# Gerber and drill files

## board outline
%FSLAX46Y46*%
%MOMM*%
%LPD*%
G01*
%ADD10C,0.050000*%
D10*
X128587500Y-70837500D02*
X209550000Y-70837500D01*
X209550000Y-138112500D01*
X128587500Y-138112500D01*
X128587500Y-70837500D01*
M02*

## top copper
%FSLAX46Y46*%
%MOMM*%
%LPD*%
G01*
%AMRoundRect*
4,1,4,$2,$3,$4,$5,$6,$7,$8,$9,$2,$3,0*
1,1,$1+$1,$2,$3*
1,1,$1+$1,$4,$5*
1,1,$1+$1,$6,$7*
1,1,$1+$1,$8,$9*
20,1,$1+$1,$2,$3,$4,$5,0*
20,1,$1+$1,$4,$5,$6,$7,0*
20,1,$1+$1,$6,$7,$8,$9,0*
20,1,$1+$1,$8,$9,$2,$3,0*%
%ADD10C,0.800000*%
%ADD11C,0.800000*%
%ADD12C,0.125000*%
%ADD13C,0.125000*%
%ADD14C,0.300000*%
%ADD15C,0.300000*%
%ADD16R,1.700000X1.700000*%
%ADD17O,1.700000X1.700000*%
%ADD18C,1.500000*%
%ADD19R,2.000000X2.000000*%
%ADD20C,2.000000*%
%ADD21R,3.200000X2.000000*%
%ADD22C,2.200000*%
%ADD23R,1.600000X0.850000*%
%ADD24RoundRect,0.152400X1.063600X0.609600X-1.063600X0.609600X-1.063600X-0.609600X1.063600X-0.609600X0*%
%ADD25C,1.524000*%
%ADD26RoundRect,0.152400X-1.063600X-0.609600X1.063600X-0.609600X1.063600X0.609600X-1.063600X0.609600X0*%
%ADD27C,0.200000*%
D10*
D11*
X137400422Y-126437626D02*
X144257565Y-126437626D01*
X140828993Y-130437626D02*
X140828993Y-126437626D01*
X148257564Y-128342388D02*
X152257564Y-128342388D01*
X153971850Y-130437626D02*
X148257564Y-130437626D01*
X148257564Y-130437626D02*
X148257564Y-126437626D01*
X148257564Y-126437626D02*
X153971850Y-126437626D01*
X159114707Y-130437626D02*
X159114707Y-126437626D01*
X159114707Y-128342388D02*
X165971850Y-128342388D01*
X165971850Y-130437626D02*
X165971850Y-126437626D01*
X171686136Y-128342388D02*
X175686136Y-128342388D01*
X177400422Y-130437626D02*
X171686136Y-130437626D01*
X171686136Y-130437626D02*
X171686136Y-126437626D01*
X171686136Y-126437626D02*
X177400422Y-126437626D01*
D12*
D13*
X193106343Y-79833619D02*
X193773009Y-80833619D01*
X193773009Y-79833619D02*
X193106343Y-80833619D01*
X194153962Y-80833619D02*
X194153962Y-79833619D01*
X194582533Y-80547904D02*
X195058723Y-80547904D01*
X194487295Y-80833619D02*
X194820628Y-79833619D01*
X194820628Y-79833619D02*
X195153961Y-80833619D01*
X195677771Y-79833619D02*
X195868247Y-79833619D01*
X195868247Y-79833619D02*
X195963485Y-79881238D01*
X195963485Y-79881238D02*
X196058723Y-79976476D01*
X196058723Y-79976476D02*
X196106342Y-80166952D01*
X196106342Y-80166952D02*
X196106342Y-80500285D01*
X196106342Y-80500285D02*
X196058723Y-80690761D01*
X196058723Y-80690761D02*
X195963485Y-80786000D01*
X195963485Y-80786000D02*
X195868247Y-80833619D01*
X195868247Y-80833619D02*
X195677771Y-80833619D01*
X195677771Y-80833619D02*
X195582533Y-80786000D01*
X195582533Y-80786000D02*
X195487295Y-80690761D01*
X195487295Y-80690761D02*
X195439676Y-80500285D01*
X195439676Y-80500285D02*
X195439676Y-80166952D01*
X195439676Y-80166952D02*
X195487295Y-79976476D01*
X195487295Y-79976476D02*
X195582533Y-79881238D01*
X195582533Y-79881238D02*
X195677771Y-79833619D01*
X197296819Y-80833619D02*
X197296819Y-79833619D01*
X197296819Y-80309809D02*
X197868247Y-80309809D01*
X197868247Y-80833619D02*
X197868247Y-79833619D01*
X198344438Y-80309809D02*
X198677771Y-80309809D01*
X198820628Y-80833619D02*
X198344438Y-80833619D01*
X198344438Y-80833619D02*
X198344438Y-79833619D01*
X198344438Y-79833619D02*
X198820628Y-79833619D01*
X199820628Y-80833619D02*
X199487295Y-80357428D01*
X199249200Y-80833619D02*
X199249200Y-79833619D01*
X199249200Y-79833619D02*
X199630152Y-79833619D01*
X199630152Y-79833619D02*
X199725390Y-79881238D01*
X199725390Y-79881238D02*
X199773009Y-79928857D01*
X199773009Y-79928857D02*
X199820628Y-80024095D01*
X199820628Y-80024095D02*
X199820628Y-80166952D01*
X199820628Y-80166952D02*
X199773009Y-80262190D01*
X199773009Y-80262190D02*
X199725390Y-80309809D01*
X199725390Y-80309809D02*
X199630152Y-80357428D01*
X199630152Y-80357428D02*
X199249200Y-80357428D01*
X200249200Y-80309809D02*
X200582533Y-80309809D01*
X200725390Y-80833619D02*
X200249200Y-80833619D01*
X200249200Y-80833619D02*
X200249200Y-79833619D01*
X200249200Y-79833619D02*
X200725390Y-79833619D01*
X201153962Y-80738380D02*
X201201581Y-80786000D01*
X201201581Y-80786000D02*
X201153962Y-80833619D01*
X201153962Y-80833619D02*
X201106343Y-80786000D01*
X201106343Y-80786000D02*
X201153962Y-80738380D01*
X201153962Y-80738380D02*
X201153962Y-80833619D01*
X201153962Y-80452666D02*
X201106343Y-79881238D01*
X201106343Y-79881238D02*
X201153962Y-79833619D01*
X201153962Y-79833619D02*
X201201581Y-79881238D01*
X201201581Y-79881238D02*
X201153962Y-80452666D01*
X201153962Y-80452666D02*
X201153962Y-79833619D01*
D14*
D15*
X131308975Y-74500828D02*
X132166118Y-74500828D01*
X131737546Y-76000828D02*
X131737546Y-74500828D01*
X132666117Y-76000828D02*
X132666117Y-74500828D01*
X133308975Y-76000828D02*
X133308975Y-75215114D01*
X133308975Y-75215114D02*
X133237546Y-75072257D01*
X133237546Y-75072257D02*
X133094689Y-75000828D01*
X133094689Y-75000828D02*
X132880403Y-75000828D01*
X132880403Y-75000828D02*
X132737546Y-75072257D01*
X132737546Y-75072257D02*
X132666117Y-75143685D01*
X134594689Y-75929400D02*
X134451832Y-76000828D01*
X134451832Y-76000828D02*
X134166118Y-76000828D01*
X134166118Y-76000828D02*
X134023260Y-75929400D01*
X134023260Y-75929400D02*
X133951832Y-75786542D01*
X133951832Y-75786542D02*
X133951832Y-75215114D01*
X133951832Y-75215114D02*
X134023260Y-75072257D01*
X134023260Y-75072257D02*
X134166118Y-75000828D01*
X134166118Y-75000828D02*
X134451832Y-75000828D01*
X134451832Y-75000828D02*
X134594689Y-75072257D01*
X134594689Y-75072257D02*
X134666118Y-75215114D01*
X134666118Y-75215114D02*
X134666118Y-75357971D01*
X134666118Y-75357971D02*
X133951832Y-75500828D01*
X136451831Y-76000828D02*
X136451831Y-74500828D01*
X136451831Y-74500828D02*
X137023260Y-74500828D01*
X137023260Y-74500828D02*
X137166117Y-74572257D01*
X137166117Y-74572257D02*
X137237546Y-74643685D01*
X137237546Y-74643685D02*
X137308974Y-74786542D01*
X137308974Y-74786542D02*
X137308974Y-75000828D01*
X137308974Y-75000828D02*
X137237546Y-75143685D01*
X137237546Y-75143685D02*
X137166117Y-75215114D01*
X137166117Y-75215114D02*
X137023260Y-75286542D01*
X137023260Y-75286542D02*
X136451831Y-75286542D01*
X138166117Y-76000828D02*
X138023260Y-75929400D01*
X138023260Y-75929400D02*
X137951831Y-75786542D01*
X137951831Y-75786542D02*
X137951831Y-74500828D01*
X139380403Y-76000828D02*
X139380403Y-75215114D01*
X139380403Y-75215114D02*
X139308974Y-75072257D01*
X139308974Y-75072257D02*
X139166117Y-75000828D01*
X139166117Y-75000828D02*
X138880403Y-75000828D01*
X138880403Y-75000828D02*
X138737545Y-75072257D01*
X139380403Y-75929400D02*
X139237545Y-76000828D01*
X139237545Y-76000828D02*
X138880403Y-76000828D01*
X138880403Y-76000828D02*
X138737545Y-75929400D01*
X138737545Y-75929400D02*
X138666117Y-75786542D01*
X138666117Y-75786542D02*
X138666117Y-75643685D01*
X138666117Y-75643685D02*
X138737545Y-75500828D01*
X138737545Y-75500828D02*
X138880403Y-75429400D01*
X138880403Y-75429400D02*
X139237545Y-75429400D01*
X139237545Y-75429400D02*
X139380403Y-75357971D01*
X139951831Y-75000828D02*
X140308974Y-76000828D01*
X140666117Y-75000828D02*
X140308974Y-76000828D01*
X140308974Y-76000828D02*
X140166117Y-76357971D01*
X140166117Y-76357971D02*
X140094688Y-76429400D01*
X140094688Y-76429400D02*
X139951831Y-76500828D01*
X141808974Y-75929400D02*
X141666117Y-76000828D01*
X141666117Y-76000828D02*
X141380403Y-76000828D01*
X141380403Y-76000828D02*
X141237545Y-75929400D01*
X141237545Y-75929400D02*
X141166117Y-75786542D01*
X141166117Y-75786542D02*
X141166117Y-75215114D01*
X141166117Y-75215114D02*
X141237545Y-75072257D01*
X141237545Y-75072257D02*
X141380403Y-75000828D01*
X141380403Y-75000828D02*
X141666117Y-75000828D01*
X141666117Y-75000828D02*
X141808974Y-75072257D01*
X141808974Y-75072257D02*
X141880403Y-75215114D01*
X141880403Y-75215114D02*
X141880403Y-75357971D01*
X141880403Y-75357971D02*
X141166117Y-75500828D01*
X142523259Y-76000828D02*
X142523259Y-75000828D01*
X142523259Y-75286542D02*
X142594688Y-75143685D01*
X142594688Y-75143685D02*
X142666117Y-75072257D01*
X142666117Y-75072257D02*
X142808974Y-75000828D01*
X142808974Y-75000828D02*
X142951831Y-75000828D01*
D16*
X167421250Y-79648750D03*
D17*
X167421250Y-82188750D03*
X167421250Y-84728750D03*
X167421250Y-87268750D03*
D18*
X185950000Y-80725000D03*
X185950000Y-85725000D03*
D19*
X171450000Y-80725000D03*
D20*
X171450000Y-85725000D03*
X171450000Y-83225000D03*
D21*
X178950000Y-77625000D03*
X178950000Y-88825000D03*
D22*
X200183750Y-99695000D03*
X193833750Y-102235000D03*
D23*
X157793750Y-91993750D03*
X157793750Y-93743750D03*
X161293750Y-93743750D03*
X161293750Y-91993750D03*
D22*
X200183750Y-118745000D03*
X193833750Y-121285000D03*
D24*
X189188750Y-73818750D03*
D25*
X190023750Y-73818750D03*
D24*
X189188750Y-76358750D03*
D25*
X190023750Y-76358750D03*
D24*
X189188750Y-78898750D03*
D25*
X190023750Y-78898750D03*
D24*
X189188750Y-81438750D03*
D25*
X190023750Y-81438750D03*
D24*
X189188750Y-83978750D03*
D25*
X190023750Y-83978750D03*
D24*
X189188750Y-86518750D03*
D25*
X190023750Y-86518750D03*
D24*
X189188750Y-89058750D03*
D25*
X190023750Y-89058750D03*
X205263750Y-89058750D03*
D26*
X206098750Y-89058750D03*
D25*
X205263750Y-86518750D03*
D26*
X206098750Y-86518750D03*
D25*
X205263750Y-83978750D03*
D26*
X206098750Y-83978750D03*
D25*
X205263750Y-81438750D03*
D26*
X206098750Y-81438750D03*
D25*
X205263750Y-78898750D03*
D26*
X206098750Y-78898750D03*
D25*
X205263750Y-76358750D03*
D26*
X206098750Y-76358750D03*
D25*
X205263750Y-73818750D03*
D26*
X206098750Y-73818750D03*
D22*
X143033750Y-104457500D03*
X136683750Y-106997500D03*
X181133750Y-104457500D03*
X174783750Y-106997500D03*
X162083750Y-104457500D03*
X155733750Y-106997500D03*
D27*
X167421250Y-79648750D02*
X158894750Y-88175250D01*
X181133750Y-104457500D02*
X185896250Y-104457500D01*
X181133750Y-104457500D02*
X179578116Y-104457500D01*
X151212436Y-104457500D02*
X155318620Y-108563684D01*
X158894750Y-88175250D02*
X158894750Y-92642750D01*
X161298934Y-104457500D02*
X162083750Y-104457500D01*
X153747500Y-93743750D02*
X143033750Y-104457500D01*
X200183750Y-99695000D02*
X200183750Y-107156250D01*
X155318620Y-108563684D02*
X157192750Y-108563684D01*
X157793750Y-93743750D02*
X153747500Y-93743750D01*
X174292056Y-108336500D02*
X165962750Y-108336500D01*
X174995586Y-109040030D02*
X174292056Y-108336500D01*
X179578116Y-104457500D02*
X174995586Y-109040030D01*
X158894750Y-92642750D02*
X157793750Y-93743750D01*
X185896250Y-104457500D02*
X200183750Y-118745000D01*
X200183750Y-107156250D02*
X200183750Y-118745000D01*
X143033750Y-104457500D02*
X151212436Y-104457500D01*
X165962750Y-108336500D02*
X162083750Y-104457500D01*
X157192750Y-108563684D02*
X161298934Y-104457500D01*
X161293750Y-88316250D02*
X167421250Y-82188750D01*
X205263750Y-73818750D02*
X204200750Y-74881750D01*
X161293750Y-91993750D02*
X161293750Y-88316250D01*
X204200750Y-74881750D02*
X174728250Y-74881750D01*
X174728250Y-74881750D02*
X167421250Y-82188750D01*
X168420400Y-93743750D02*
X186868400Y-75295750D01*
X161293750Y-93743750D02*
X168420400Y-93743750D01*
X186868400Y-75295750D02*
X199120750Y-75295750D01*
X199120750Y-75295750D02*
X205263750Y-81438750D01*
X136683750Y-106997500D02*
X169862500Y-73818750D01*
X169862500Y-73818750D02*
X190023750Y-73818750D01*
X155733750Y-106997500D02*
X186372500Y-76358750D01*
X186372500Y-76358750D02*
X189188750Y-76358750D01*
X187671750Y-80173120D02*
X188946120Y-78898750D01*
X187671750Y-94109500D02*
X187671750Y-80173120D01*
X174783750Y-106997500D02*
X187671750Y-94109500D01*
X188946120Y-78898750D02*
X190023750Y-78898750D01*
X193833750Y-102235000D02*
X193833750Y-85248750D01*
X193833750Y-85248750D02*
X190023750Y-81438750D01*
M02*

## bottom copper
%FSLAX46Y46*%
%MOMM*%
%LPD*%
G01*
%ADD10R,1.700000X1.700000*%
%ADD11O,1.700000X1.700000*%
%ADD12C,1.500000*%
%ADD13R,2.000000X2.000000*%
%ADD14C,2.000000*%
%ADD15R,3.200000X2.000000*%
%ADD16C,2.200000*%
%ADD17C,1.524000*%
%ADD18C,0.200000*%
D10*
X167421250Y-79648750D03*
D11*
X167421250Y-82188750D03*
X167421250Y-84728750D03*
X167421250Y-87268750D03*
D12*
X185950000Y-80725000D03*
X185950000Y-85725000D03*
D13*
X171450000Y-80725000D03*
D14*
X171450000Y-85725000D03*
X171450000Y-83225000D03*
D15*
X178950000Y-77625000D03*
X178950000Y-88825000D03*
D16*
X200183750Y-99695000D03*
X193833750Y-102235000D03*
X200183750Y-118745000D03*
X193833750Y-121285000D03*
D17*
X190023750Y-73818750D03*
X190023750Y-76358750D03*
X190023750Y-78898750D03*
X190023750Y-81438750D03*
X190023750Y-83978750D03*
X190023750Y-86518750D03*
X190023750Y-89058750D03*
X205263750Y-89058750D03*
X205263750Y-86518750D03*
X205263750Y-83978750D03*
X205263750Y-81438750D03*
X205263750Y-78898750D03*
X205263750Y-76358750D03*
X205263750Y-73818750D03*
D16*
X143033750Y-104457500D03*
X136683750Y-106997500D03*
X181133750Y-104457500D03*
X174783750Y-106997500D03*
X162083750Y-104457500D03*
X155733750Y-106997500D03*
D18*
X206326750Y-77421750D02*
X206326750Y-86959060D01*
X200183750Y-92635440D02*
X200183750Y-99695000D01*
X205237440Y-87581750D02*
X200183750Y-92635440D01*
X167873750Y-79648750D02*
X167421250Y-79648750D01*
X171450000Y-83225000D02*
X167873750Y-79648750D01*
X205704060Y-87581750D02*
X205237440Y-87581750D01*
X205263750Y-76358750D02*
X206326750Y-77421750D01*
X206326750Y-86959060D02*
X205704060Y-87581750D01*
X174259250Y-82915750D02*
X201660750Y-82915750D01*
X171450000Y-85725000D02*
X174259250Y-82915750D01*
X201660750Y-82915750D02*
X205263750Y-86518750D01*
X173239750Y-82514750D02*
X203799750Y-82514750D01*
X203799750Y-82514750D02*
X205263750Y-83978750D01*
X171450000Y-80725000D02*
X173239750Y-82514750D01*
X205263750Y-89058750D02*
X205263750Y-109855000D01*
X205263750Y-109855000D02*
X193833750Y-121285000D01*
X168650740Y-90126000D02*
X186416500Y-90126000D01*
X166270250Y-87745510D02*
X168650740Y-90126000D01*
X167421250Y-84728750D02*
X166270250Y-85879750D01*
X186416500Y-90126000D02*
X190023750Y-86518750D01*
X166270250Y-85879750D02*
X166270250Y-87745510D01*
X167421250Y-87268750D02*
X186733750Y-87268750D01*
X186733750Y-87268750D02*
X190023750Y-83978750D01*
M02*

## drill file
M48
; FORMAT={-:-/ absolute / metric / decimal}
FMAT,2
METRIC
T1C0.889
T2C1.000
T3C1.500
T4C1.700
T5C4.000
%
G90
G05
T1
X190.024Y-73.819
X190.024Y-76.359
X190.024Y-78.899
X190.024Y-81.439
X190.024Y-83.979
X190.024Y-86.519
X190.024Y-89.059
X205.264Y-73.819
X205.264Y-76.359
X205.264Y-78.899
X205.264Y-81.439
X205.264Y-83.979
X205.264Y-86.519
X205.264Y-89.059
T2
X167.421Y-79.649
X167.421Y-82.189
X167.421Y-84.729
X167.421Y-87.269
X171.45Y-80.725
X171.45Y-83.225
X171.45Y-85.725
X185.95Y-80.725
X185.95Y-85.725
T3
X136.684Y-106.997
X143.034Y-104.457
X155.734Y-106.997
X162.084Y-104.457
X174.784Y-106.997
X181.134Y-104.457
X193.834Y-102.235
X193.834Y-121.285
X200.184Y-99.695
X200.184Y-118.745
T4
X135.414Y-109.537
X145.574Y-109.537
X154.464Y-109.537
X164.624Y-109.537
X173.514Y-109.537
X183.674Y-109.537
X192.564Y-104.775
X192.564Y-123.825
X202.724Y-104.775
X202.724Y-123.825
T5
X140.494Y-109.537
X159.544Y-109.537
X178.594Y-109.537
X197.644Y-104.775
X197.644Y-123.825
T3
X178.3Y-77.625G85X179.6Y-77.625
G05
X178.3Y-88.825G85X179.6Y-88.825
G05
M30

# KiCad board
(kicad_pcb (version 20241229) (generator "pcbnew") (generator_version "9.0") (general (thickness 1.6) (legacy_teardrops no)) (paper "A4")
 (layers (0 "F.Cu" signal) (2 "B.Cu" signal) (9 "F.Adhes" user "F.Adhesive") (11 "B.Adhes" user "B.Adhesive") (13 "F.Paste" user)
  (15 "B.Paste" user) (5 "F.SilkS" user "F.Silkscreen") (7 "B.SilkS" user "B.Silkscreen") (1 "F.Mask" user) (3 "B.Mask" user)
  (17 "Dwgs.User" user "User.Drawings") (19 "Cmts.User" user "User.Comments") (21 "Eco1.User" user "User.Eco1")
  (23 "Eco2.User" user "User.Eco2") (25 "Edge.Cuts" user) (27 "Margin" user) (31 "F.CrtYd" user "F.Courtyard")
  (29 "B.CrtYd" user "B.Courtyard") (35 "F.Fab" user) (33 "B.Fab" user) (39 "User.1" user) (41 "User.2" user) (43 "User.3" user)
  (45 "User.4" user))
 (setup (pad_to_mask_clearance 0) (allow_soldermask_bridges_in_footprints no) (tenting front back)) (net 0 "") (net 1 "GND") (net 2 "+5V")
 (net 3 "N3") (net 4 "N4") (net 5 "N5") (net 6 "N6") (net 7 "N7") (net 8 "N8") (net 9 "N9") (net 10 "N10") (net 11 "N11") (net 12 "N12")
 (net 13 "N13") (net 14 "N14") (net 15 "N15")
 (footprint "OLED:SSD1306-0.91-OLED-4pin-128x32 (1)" (layer "F.Cu") (at 130.92125 77.45875)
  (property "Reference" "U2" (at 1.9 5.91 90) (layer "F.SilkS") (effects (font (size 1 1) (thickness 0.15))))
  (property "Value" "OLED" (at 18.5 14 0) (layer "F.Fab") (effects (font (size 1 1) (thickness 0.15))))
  (pad "1" thru_hole rect (at 36.5 2.19) (size 1.7 1.7) (drill 1) (layers "*.Cu" "*.Mask") (remove_unused_layers no) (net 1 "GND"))
  (pad "2" thru_hole oval (at 36.5 4.73) (size 1.7 1.7) (drill 1) (layers "*.Cu" "*.Mask") (remove_unused_layers no) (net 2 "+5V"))
  (pad "3" thru_hole oval (at 36.5 7.27) (size 1.7 1.7) (drill 1) (layers "*.Cu" "*.Mask") (remove_unused_layers no) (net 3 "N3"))
  (pad "4" thru_hole oval (at 36.5 9.81) (size 1.7 1.7) (drill 1) (layers "*.Cu" "*.Mask") (remove_unused_layers no) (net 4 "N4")))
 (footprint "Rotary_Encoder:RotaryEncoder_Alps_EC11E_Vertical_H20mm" (layer "F.Cu") (at 171.45 80.725)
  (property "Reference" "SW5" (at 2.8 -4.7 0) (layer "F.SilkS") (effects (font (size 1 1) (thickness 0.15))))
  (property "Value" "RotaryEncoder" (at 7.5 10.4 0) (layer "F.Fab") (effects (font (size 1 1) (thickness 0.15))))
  (pad "" thru_hole circle (at 14.5 0) (size 1.5 1.5) (drill 1) (layers "*.Cu" "*.Mask") (remove_unused_layers no))
  (pad "" thru_hole circle (at 14.5 5) (size 1.5 1.5) (drill 1) (layers "*.Cu" "*.Mask") (remove_unused_layers no))
  (pad "A" thru_hole rect (at 0 0) (size 2 2) (drill 1) (layers "*.Cu" "*.Mask") (remove_unused_layers no) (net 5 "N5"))
  (pad "B" thru_hole circle (at 0 5) (size 2 2) (drill 1) (layers "*.Cu" "*.Mask") (remove_unused_layers no) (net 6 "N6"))
  (pad "C" thru_hole circle (at 0 2.5) (size 2 2) (drill 1) (layers "*.Cu" "*.Mask") (remove_unused_layers no) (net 1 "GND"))
  (pad "MP" thru_hole rect (at 7.5 -3.1) (size 3.2 2) (drill oval 2.8 1.5) (layers "*.Cu" "*.Mask") (remove_unused_layers no))
  (pad "MP" thru_hole rect (at 7.5 8.1) (size 3.2 2) (drill oval 2.8 1.5) (layers "*.Cu" "*.Mask") (remove_unused_layers no)))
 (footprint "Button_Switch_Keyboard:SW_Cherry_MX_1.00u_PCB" (layer "F.Cu") (at 200.18375 99.695)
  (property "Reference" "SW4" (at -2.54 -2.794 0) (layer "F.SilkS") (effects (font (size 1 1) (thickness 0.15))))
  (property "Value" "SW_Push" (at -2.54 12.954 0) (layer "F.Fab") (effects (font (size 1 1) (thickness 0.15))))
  (pad "" np_thru_hole circle (at -7.62 5.08) (size 1.7 1.7) (drill 1.7) (layers "*.Cu" "*.Mask"))
  (pad "" np_thru_hole circle (at -2.54 5.08) (size 4 4) (drill 4) (layers "*.Cu" "*.Mask"))
  (pad "" np_thru_hole circle (at 2.54 5.08) (size 1.7 1.7) (drill 1.7) (layers "*.Cu" "*.Mask"))
  (pad "1" thru_hole circle (at 0 0) (size 2.2 2.2) (drill 1.5) (layers "*.Cu" "*.Mask") (remove_unused_layers no) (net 1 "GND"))
  (pad "2" thru_hole circle (at -6.35 2.54) (size 2.2 2.2) (drill 1.5) (layers "*.Cu" "*.Mask") (remove_unused_layers no) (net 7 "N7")))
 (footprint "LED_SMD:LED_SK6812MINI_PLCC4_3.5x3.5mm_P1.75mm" (layer "F.Cu") (at 159.54375 92.86875)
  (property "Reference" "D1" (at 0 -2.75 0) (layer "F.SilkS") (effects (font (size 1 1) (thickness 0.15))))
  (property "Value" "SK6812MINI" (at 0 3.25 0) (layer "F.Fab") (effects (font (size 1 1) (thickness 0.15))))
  (pad "1" smd rect (at -1.75 -0.875) (size 1.6 0.85) (layers "F.Cu" "F.Mask" "F.Paste") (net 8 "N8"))
  (pad "2" smd rect (at -1.75 0.875) (size 1.6 0.85) (layers "F.Cu" "F.Mask" "F.Paste") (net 1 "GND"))
  (pad "3" smd rect (at 1.75 0.875) (size 1.6 0.85) (layers "F.Cu" "F.Mask" "F.Paste") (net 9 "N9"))
  (pad "4" smd rect (at 1.75 -0.875) (size 1.6 0.85) (layers "F.Cu" "F.Mask" "F.Paste") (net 2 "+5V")))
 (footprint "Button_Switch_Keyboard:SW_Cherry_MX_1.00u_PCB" (layer "F.Cu") (at 200.18375 118.745)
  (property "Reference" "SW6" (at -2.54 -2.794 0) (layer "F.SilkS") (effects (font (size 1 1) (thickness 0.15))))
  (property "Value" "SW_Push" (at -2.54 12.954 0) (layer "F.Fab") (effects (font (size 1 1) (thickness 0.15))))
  (pad "" np_thru_hole circle (at -7.62 5.08) (size 1.7 1.7) (drill 1.7) (layers "*.Cu" "*.Mask"))
  (pad "" np_thru_hole circle (at -2.54 5.08) (size 4 4) (drill 4) (layers "*.Cu" "*.Mask"))
  (pad "" np_thru_hole circle (at 2.54 5.08) (size 1.7 1.7) (drill 1.7) (layers "*.Cu" "*.Mask"))
  (pad "1" thru_hole circle (at 0 0) (size 2.2 2.2) (drill 1.5) (layers "*.Cu" "*.Mask") (remove_unused_layers no) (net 1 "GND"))
  (pad "2" thru_hole circle (at -6.35 2.54) (size 2.2 2.2) (drill 1.5) (layers "*.Cu" "*.Mask") (remove_unused_layers no) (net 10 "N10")))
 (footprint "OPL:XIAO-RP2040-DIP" (layer "F.Cu") (at 197.64375 81.43875)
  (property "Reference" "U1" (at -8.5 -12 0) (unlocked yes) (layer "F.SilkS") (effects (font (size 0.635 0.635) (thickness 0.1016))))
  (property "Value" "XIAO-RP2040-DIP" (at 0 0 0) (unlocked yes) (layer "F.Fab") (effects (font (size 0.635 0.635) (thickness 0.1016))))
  (pad "1" smd roundrect (at -8.455 -7.62 180) (size 2.432 1.524) (layers "F.Cu" "F.Mask") (roundrect_rratio 0.1) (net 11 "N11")
   (thermal_bridge_angle 45))
  (pad "1" thru_hole circle (at -7.62 -7.62 180) (size 1.524 1.524) (drill 0.889) (layers "*.Cu" "*.Mask") (remove_unused_layers no)
   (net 11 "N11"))
  (pad "2" smd roundrect (at -8.455 -5.08 180) (size 2.432 1.524) (layers "F.Cu" "F.Mask") (roundrect_rratio 0.1) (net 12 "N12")
   (thermal_bridge_angle 45))
  (pad "2" thru_hole circle (at -7.62 -5.08 180) (size 1.524 1.524) (drill 0.889) (layers "*.Cu" "*.Mask") (remove_unused_layers no)
   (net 12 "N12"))
  (pad "3" smd roundrect (at -8.455 -2.54 180) (size 2.432 1.524) (layers "F.Cu" "F.Mask") (roundrect_rratio 0.1) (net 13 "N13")
   (thermal_bridge_angle 45))
  (pad "3" thru_hole circle (at -7.62 -2.54 180) (size 1.524 1.524) (drill 0.889) (layers "*.Cu" "*.Mask") (remove_unused_layers no)
   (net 13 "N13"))
  (pad "4" smd roundrect (at -8.455 0 180) (size 2.432 1.524) (layers "F.Cu" "F.Mask") (roundrect_rratio 0.1) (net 7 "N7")
   (thermal_bridge_angle 45))
  (pad "4" thru_hole circle (at -7.62 0 180) (size 1.524 1.524) (drill 0.889) (layers "*.Cu" "*.Mask") (remove_unused_layers no)
   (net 7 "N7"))
  (pad "5" smd roundrect (at -8.455 2.54 180) (size 2.432 1.524) (layers "F.Cu" "F.Mask") (roundrect_rratio 0.1) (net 4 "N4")
   (thermal_bridge_angle 45))
  (pad "5" thru_hole circle (at -7.62 2.54 180) (size 1.524 1.524) (drill 0.889) (layers "*.Cu" "*.Mask") (remove_unused_layers no)
   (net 4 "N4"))
  (pad "6" smd roundrect (at -8.455 5.08 180) (size 2.432 1.524) (layers "F.Cu" "F.Mask") (roundrect_rratio 0.1) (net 3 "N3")
   (thermal_bridge_angle 45))
  (pad "6" thru_hole circle (at -7.62 5.08 180) (size 1.524 1.524) (drill 0.889) (layers "*.Cu" "*.Mask") (remove_unused_layers no)
   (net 3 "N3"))
  (pad "7" smd roundrect (at -8.455 7.62 180) (size 2.432 1.524) (layers "F.Cu" "F.Mask") (roundrect_rratio 0.1) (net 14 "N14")
   (thermal_bridge_angle 45))
  (pad "7" thru_hole circle (at -7.62 7.62 180) (size 1.524 1.524) (drill 0.889) (layers "*.Cu" "*.Mask") (remove_unused_layers no)
   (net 14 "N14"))
  (pad "8" thru_hole circle (at 7.62 7.62) (size 1.524 1.524) (drill 0.889) (layers "*.Cu" "*.Mask") (remove_unused_layers no)
   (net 10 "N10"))
  (pad "8" smd roundrect (at 8.455 7.62) (size 2.432 1.524) (layers "F.Cu" "F.Mask") (roundrect_rratio 0.1) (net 10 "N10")
   (thermal_bridge_angle 45))
  (pad "9" thru_hole circle (at 7.62 5.08) (size 1.524 1.524) (drill 0.889) (layers "*.Cu" "*.Mask") (remove_unused_layers no) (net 6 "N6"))
  (pad "9" smd roundrect (at 8.455 5.08) (size 2.432 1.524) (layers "F.Cu" "F.Mask") (roundrect_rratio 0.1) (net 6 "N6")
   (thermal_bridge_angle 45))
  (pad "10" thru_hole circle (at 7.62 2.54) (size 1.524 1.524) (drill 0.889) (layers "*.Cu" "*.Mask") (remove_unused_layers no) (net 5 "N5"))
  (pad "10" smd roundrect (at 8.455 2.54) (size 2.432 1.524) (layers "F.Cu" "F.Mask") (roundrect_rratio 0.1) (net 5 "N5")
   (thermal_bridge_angle 45))
  (pad "11" thru_hole circle (at 7.62 0) (size 1.524 1.524) (drill 0.889) (layers "*.Cu" "*.Mask") (remove_unused_layers no) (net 9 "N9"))
  (pad "11" smd roundrect (at 8.455 0) (size 2.432 1.524) (layers "F.Cu" "F.Mask") (roundrect_rratio 0.1) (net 9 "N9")
   (thermal_bridge_angle 45))
  (pad "12" thru_hole circle (at 7.62 -2.54) (size 1.524 1.524) (drill 0.889) (layers "*.Cu" "*.Mask") (remove_unused_layers no)
   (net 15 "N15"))
  (pad "12" smd roundrect (at 8.455 -2.54) (size 2.432 1.524) (layers "F.Cu" "F.Mask") (roundrect_rratio 0.1) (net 15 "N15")
   (thermal_bridge_angle 45))
  (pad "13" thru_hole circle (at 7.62 -5.08) (size 1.524 1.524) (drill 0.889) (layers "*.Cu" "*.Mask") (remove_unused_layers no)
   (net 1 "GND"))
  (pad "13" smd roundrect (at 8.455 -5.08) (size 2.432 1.524) (layers "F.Cu" "F.Mask") (roundrect_rratio 0.1) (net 1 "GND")
   (thermal_bridge_angle 45))
  (pad "14" thru_hole circle (at 7.62 -7.62) (size 1.524 1.524) (drill 0.889) (layers "*.Cu" "*.Mask") (remove_unused_layers no)
   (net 2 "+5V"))
  (pad "14" smd roundrect (at 8.455 -7.62) (size 2.432 1.524) (layers "F.Cu" "F.Mask") (roundrect_rratio 0.1) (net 2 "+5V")
   (thermal_bridge_angle 45)))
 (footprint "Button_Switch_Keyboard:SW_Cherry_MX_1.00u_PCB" (layer "F.Cu") (at 143.03375 104.4575)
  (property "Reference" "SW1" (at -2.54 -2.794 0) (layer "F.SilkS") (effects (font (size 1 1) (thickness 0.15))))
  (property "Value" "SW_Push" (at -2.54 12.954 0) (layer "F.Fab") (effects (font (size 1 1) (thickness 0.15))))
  (pad "" np_thru_hole circle (at -7.62 5.08) (size 1.7 1.7) (drill 1.7) (layers "*.Cu" "*.Mask"))
  (pad "" np_thru_hole circle (at -2.54 5.08) (size 4 4) (drill 4) (layers "*.Cu" "*.Mask"))
  (pad "" np_thru_hole circle (at 2.54 5.08) (size 1.7 1.7) (drill 1.7) (layers "*.Cu" "*.Mask"))
  (pad "1" thru_hole circle (at 0 0) (size 2.2 2.2) (drill 1.5) (layers "*.Cu" "*.Mask") (remove_unused_layers no) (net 1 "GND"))
  (pad "2" thru_hole circle (at -6.35 2.54) (size 2.2 2.2) (drill 1.5) (layers "*.Cu" "*.Mask") (remove_unused_layers no) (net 11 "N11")))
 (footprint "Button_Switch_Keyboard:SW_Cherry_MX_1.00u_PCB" (layer "F.Cu") (at 181.13375 104.4575)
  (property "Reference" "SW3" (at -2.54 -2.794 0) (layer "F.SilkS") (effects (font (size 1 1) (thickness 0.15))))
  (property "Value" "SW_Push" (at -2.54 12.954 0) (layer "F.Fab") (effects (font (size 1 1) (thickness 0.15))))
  (pad "" np_thru_hole circle (at -7.62 5.08) (size 1.7 1.7) (drill 1.7) (layers "*.Cu" "*.Mask"))
  (pad "" np_thru_hole circle (at -2.54 5.08) (size 4 4) (drill 4) (layers "*.Cu" "*.Mask"))
  (pad "" np_thru_hole circle (at 2.54 5.08) (size 1.7 1.7) (drill 1.7) (layers "*.Cu" "*.Mask"))
  (pad "1" thru_hole circle (at 0 0) (size 2.2 2.2) (drill 1.5) (layers "*.Cu" "*.Mask") (remove_unused_layers no) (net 1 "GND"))
  (pad "2" thru_hole circle (at -6.35 2.54) (size 2.2 2.2) (drill 1.5) (layers "*.Cu" "*.Mask") (remove_unused_layers no) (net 13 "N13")))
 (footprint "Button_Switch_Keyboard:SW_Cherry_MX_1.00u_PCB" (layer "F.Cu") (at 162.08375 104.4575)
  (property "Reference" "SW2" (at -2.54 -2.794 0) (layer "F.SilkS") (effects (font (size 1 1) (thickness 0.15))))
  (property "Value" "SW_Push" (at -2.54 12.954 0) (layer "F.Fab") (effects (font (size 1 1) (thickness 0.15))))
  (pad "" np_thru_hole circle (at -7.62 5.08) (size 1.7 1.7) (drill 1.7) (layers "*.Cu" "*.Mask"))
  (pad "" np_thru_hole circle (at -2.54 5.08) (size 4 4) (drill 4) (layers "*.Cu" "*.Mask"))
  (pad "" np_thru_hole circle (at 2.54 5.08) (size 1.7 1.7) (drill 1.7) (layers "*.Cu" "*.Mask"))
  (pad "1" thru_hole circle (at 0 0) (size 2.2 2.2) (drill 1.5) (layers "*.Cu" "*.Mask") (remove_unused_layers no) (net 1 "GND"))
  (pad "2" thru_hole circle (at -6.35 2.54) (size 2.2 2.2) (drill 1.5) (layers "*.Cu" "*.Mask") (remove_unused_layers no) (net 12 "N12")))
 (gr_rect (start 128.5875 70.8375) (end 209.55 138.1125) (stroke (width 0.05) (type solid)) (fill no) (layer "Edge.Cuts"))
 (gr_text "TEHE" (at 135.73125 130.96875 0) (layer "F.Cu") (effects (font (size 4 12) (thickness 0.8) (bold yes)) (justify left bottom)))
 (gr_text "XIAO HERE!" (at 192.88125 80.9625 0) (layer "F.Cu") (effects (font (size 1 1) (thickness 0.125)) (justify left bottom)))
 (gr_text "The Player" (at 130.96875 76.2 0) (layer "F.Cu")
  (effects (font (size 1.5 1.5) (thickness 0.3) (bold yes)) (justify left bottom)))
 (segment (start 167.42125 79.64875) (end 158.89475 88.17525) (width 0.2) (layer "F.Cu") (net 1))
 (segment (start 181.13375 104.4575) (end 185.89625 104.4575) (width 0.2) (layer "F.Cu") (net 1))
 (segment (start 181.13375 104.4575) (end 179.578116 104.4575) (width 0.2) (layer "F.Cu") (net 1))
 (segment (start 151.212436 104.4575) (end 155.31862 108.563684) (width 0.2) (layer "F.Cu") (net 1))
 (segment (start 158.89475 88.17525) (end 158.89475 92.64275) (width 0.2) (layer "F.Cu") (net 1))
 (segment (start 161.298934 104.4575) (end 162.08375 104.4575) (width 0.2) (layer "F.Cu") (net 1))
 (segment (start 153.7475 93.74375) (end 143.03375 104.4575) (width 0.2) (layer "F.Cu") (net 1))
 (segment (start 200.18375 99.695) (end 200.18375 107.15625) (width 0.2) (layer "F.Cu") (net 1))
 (segment (start 155.31862 108.563684) (end 157.19275 108.563684) (width 0.2) (layer "F.Cu") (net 1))
 (segment (start 157.79375 93.74375) (end 153.7475 93.74375) (width 0.2) (layer "F.Cu") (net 1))
 (segment (start 174.292056 108.3365) (end 165.96275 108.3365) (width 0.2) (layer "F.Cu") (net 1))
 (segment (start 174.995586 109.04003) (end 174.292056 108.3365) (width 0.2) (layer "F.Cu") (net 1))
 (segment (start 179.578116 104.4575) (end 174.995586 109.04003) (width 0.2) (layer "F.Cu") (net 1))
 (segment (start 158.89475 92.64275) (end 157.79375 93.74375) (width 0.2) (layer "F.Cu") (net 1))
 (segment (start 185.89625 104.4575) (end 200.18375 118.745) (width 0.2) (layer "F.Cu") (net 1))
 (segment (start 200.18375 107.15625) (end 200.18375 118.745) (width 0.2) (layer "F.Cu") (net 1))
 (segment (start 143.03375 104.4575) (end 151.212436 104.4575) (width 0.2) (layer "F.Cu") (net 1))
 (segment (start 165.96275 108.3365) (end 162.08375 104.4575) (width 0.2) (layer "F.Cu") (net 1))
 (segment (start 157.19275 108.563684) (end 161.298934 104.4575) (width 0.2) (layer "F.Cu") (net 1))
 (segment (start 206.32675 77.42175) (end 206.32675 86.95906) (width 0.2) (layer "B.Cu") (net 1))
 (segment (start 200.18375 92.63544) (end 200.18375 99.695) (width 0.2) (layer "B.Cu") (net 1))
 (segment (start 205.23744 87.58175) (end 200.18375 92.63544) (width 0.2) (layer "B.Cu") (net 1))
 (segment (start 167.87375 79.64875) (end 167.42125 79.64875) (width 0.2) (layer "B.Cu") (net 1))
 (segment (start 171.45 83.225) (end 167.87375 79.64875) (width 0.2) (layer "B.Cu") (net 1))
 (segment (start 205.70406 87.58175) (end 205.23744 87.58175) (width 0.2) (layer "B.Cu") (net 1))
 (segment (start 205.26375 76.35875) (end 206.32675 77.42175) (width 0.2) (layer "B.Cu") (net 1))
 (segment (start 206.32675 86.95906) (end 205.70406 87.58175) (width 0.2) (layer "B.Cu") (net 1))
 (segment (start 161.29375 88.31625) (end 167.42125 82.18875) (width 0.2) (layer "F.Cu") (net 2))
 (segment (start 205.26375 73.81875) (end 204.20075 74.88175) (width 0.2) (layer "F.Cu") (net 2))
 (segment (start 161.29375 91.99375) (end 161.29375 88.31625) (width 0.2) (layer "F.Cu") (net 2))
 (segment (start 204.20075 74.88175) (end 174.72825 74.88175) (width 0.2) (layer "F.Cu") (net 2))
 (segment (start 174.72825 74.88175) (end 167.42125 82.18875) (width 0.2) (layer "F.Cu") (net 2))
 (segment (start 168.4204 93.74375) (end 186.8684 75.29575) (width 0.2) (layer "F.Cu") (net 9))
 (segment (start 161.29375 93.74375) (end 168.4204 93.74375) (width 0.2) (layer "F.Cu") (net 9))
 (segment (start 186.8684 75.29575) (end 199.12075 75.29575) (width 0.2) (layer "F.Cu") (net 9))
 (segment (start 199.12075 75.29575) (end 205.26375 81.43875) (width 0.2) (layer "F.Cu") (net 9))
 (segment (start 136.68375 106.9975) (end 169.8625 73.81875) (width 0.2) (layer "F.Cu") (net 11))
 (segment (start 169.8625 73.81875) (end 190.02375 73.81875) (width 0.2) (layer "F.Cu") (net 11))
 (segment (start 155.73375 106.9975) (end 186.3725 76.35875) (width 0.2) (layer "F.Cu") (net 12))
 (segment (start 186.3725 76.35875) (end 189.18875 76.35875) (width 0.2) (layer "F.Cu") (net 12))
 (segment (start 187.67175 80.17312) (end 188.94612 78.89875) (width 0.2) (layer "F.Cu") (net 13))
 (segment (start 187.67175 94.1095) (end 187.67175 80.17312) (width 0.2) (layer "F.Cu") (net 13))
 (segment (start 174.78375 106.9975) (end 187.67175 94.1095) (width 0.2) (layer "F.Cu") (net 13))
 (segment (start 188.94612 78.89875) (end 190.02375 78.89875) (width 0.2) (layer "F.Cu") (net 13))
 (segment (start 193.83375 102.235) (end 193.83375 85.24875) (width 0.2) (layer "F.Cu") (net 7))
 (segment (start 193.83375 85.24875) (end 190.02375 81.43875) (width 0.2) (layer "F.Cu") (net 7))
 (segment (start 174.25925 82.91575) (end 201.66075 82.91575) (width 0.2) (layer "B.Cu") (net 6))
 (segment (start 171.45 85.725) (end 174.25925 82.91575) (width 0.2) (layer "B.Cu") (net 6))
 (segment (start 201.66075 82.91575) (end 205.26375 86.51875) (width 0.2) (layer "B.Cu") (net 6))
 (segment (start 173.23975 82.51475) (end 203.79975 82.51475) (width 0.2) (layer "B.Cu") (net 5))
 (segment (start 203.79975 82.51475) (end 205.26375 83.97875) (width 0.2) (layer "B.Cu") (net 5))
 (segment (start 171.45 80.725) (end 173.23975 82.51475) (width 0.2) (layer "B.Cu") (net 5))
 (segment (start 205.26375 89.05875) (end 205.26375 109.855) (width 0.2) (layer "B.Cu") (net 10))
 (segment (start 205.26375 109.855) (end 193.83375 121.285) (width 0.2) (layer "B.Cu") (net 10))
 (segment (start 168.65074 90.126) (end 186.4165 90.126) (width 0.2) (layer "B.Cu") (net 3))
 (segment (start 166.27025 87.74551) (end 168.65074 90.126) (width 0.2) (layer "B.Cu") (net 3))
 (segment (start 167.42125 84.72875) (end 166.27025 85.87975) (width 0.2) (layer "B.Cu") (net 3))
 (segment (start 186.4165 90.126) (end 190.02375 86.51875) (width 0.2) (layer "B.Cu") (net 3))
 (segment (start 166.27025 85.87975) (end 166.27025 87.74551) (width 0.2) (layer "B.Cu") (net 3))
 (segment (start 167.42125 87.26875) (end 186.73375 87.26875) (width 0.2) (layer "B.Cu") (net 4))
 (segment (start 186.73375 87.26875) (end 190.02375 83.97875) (width 0.2) (layer "B.Cu") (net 4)))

